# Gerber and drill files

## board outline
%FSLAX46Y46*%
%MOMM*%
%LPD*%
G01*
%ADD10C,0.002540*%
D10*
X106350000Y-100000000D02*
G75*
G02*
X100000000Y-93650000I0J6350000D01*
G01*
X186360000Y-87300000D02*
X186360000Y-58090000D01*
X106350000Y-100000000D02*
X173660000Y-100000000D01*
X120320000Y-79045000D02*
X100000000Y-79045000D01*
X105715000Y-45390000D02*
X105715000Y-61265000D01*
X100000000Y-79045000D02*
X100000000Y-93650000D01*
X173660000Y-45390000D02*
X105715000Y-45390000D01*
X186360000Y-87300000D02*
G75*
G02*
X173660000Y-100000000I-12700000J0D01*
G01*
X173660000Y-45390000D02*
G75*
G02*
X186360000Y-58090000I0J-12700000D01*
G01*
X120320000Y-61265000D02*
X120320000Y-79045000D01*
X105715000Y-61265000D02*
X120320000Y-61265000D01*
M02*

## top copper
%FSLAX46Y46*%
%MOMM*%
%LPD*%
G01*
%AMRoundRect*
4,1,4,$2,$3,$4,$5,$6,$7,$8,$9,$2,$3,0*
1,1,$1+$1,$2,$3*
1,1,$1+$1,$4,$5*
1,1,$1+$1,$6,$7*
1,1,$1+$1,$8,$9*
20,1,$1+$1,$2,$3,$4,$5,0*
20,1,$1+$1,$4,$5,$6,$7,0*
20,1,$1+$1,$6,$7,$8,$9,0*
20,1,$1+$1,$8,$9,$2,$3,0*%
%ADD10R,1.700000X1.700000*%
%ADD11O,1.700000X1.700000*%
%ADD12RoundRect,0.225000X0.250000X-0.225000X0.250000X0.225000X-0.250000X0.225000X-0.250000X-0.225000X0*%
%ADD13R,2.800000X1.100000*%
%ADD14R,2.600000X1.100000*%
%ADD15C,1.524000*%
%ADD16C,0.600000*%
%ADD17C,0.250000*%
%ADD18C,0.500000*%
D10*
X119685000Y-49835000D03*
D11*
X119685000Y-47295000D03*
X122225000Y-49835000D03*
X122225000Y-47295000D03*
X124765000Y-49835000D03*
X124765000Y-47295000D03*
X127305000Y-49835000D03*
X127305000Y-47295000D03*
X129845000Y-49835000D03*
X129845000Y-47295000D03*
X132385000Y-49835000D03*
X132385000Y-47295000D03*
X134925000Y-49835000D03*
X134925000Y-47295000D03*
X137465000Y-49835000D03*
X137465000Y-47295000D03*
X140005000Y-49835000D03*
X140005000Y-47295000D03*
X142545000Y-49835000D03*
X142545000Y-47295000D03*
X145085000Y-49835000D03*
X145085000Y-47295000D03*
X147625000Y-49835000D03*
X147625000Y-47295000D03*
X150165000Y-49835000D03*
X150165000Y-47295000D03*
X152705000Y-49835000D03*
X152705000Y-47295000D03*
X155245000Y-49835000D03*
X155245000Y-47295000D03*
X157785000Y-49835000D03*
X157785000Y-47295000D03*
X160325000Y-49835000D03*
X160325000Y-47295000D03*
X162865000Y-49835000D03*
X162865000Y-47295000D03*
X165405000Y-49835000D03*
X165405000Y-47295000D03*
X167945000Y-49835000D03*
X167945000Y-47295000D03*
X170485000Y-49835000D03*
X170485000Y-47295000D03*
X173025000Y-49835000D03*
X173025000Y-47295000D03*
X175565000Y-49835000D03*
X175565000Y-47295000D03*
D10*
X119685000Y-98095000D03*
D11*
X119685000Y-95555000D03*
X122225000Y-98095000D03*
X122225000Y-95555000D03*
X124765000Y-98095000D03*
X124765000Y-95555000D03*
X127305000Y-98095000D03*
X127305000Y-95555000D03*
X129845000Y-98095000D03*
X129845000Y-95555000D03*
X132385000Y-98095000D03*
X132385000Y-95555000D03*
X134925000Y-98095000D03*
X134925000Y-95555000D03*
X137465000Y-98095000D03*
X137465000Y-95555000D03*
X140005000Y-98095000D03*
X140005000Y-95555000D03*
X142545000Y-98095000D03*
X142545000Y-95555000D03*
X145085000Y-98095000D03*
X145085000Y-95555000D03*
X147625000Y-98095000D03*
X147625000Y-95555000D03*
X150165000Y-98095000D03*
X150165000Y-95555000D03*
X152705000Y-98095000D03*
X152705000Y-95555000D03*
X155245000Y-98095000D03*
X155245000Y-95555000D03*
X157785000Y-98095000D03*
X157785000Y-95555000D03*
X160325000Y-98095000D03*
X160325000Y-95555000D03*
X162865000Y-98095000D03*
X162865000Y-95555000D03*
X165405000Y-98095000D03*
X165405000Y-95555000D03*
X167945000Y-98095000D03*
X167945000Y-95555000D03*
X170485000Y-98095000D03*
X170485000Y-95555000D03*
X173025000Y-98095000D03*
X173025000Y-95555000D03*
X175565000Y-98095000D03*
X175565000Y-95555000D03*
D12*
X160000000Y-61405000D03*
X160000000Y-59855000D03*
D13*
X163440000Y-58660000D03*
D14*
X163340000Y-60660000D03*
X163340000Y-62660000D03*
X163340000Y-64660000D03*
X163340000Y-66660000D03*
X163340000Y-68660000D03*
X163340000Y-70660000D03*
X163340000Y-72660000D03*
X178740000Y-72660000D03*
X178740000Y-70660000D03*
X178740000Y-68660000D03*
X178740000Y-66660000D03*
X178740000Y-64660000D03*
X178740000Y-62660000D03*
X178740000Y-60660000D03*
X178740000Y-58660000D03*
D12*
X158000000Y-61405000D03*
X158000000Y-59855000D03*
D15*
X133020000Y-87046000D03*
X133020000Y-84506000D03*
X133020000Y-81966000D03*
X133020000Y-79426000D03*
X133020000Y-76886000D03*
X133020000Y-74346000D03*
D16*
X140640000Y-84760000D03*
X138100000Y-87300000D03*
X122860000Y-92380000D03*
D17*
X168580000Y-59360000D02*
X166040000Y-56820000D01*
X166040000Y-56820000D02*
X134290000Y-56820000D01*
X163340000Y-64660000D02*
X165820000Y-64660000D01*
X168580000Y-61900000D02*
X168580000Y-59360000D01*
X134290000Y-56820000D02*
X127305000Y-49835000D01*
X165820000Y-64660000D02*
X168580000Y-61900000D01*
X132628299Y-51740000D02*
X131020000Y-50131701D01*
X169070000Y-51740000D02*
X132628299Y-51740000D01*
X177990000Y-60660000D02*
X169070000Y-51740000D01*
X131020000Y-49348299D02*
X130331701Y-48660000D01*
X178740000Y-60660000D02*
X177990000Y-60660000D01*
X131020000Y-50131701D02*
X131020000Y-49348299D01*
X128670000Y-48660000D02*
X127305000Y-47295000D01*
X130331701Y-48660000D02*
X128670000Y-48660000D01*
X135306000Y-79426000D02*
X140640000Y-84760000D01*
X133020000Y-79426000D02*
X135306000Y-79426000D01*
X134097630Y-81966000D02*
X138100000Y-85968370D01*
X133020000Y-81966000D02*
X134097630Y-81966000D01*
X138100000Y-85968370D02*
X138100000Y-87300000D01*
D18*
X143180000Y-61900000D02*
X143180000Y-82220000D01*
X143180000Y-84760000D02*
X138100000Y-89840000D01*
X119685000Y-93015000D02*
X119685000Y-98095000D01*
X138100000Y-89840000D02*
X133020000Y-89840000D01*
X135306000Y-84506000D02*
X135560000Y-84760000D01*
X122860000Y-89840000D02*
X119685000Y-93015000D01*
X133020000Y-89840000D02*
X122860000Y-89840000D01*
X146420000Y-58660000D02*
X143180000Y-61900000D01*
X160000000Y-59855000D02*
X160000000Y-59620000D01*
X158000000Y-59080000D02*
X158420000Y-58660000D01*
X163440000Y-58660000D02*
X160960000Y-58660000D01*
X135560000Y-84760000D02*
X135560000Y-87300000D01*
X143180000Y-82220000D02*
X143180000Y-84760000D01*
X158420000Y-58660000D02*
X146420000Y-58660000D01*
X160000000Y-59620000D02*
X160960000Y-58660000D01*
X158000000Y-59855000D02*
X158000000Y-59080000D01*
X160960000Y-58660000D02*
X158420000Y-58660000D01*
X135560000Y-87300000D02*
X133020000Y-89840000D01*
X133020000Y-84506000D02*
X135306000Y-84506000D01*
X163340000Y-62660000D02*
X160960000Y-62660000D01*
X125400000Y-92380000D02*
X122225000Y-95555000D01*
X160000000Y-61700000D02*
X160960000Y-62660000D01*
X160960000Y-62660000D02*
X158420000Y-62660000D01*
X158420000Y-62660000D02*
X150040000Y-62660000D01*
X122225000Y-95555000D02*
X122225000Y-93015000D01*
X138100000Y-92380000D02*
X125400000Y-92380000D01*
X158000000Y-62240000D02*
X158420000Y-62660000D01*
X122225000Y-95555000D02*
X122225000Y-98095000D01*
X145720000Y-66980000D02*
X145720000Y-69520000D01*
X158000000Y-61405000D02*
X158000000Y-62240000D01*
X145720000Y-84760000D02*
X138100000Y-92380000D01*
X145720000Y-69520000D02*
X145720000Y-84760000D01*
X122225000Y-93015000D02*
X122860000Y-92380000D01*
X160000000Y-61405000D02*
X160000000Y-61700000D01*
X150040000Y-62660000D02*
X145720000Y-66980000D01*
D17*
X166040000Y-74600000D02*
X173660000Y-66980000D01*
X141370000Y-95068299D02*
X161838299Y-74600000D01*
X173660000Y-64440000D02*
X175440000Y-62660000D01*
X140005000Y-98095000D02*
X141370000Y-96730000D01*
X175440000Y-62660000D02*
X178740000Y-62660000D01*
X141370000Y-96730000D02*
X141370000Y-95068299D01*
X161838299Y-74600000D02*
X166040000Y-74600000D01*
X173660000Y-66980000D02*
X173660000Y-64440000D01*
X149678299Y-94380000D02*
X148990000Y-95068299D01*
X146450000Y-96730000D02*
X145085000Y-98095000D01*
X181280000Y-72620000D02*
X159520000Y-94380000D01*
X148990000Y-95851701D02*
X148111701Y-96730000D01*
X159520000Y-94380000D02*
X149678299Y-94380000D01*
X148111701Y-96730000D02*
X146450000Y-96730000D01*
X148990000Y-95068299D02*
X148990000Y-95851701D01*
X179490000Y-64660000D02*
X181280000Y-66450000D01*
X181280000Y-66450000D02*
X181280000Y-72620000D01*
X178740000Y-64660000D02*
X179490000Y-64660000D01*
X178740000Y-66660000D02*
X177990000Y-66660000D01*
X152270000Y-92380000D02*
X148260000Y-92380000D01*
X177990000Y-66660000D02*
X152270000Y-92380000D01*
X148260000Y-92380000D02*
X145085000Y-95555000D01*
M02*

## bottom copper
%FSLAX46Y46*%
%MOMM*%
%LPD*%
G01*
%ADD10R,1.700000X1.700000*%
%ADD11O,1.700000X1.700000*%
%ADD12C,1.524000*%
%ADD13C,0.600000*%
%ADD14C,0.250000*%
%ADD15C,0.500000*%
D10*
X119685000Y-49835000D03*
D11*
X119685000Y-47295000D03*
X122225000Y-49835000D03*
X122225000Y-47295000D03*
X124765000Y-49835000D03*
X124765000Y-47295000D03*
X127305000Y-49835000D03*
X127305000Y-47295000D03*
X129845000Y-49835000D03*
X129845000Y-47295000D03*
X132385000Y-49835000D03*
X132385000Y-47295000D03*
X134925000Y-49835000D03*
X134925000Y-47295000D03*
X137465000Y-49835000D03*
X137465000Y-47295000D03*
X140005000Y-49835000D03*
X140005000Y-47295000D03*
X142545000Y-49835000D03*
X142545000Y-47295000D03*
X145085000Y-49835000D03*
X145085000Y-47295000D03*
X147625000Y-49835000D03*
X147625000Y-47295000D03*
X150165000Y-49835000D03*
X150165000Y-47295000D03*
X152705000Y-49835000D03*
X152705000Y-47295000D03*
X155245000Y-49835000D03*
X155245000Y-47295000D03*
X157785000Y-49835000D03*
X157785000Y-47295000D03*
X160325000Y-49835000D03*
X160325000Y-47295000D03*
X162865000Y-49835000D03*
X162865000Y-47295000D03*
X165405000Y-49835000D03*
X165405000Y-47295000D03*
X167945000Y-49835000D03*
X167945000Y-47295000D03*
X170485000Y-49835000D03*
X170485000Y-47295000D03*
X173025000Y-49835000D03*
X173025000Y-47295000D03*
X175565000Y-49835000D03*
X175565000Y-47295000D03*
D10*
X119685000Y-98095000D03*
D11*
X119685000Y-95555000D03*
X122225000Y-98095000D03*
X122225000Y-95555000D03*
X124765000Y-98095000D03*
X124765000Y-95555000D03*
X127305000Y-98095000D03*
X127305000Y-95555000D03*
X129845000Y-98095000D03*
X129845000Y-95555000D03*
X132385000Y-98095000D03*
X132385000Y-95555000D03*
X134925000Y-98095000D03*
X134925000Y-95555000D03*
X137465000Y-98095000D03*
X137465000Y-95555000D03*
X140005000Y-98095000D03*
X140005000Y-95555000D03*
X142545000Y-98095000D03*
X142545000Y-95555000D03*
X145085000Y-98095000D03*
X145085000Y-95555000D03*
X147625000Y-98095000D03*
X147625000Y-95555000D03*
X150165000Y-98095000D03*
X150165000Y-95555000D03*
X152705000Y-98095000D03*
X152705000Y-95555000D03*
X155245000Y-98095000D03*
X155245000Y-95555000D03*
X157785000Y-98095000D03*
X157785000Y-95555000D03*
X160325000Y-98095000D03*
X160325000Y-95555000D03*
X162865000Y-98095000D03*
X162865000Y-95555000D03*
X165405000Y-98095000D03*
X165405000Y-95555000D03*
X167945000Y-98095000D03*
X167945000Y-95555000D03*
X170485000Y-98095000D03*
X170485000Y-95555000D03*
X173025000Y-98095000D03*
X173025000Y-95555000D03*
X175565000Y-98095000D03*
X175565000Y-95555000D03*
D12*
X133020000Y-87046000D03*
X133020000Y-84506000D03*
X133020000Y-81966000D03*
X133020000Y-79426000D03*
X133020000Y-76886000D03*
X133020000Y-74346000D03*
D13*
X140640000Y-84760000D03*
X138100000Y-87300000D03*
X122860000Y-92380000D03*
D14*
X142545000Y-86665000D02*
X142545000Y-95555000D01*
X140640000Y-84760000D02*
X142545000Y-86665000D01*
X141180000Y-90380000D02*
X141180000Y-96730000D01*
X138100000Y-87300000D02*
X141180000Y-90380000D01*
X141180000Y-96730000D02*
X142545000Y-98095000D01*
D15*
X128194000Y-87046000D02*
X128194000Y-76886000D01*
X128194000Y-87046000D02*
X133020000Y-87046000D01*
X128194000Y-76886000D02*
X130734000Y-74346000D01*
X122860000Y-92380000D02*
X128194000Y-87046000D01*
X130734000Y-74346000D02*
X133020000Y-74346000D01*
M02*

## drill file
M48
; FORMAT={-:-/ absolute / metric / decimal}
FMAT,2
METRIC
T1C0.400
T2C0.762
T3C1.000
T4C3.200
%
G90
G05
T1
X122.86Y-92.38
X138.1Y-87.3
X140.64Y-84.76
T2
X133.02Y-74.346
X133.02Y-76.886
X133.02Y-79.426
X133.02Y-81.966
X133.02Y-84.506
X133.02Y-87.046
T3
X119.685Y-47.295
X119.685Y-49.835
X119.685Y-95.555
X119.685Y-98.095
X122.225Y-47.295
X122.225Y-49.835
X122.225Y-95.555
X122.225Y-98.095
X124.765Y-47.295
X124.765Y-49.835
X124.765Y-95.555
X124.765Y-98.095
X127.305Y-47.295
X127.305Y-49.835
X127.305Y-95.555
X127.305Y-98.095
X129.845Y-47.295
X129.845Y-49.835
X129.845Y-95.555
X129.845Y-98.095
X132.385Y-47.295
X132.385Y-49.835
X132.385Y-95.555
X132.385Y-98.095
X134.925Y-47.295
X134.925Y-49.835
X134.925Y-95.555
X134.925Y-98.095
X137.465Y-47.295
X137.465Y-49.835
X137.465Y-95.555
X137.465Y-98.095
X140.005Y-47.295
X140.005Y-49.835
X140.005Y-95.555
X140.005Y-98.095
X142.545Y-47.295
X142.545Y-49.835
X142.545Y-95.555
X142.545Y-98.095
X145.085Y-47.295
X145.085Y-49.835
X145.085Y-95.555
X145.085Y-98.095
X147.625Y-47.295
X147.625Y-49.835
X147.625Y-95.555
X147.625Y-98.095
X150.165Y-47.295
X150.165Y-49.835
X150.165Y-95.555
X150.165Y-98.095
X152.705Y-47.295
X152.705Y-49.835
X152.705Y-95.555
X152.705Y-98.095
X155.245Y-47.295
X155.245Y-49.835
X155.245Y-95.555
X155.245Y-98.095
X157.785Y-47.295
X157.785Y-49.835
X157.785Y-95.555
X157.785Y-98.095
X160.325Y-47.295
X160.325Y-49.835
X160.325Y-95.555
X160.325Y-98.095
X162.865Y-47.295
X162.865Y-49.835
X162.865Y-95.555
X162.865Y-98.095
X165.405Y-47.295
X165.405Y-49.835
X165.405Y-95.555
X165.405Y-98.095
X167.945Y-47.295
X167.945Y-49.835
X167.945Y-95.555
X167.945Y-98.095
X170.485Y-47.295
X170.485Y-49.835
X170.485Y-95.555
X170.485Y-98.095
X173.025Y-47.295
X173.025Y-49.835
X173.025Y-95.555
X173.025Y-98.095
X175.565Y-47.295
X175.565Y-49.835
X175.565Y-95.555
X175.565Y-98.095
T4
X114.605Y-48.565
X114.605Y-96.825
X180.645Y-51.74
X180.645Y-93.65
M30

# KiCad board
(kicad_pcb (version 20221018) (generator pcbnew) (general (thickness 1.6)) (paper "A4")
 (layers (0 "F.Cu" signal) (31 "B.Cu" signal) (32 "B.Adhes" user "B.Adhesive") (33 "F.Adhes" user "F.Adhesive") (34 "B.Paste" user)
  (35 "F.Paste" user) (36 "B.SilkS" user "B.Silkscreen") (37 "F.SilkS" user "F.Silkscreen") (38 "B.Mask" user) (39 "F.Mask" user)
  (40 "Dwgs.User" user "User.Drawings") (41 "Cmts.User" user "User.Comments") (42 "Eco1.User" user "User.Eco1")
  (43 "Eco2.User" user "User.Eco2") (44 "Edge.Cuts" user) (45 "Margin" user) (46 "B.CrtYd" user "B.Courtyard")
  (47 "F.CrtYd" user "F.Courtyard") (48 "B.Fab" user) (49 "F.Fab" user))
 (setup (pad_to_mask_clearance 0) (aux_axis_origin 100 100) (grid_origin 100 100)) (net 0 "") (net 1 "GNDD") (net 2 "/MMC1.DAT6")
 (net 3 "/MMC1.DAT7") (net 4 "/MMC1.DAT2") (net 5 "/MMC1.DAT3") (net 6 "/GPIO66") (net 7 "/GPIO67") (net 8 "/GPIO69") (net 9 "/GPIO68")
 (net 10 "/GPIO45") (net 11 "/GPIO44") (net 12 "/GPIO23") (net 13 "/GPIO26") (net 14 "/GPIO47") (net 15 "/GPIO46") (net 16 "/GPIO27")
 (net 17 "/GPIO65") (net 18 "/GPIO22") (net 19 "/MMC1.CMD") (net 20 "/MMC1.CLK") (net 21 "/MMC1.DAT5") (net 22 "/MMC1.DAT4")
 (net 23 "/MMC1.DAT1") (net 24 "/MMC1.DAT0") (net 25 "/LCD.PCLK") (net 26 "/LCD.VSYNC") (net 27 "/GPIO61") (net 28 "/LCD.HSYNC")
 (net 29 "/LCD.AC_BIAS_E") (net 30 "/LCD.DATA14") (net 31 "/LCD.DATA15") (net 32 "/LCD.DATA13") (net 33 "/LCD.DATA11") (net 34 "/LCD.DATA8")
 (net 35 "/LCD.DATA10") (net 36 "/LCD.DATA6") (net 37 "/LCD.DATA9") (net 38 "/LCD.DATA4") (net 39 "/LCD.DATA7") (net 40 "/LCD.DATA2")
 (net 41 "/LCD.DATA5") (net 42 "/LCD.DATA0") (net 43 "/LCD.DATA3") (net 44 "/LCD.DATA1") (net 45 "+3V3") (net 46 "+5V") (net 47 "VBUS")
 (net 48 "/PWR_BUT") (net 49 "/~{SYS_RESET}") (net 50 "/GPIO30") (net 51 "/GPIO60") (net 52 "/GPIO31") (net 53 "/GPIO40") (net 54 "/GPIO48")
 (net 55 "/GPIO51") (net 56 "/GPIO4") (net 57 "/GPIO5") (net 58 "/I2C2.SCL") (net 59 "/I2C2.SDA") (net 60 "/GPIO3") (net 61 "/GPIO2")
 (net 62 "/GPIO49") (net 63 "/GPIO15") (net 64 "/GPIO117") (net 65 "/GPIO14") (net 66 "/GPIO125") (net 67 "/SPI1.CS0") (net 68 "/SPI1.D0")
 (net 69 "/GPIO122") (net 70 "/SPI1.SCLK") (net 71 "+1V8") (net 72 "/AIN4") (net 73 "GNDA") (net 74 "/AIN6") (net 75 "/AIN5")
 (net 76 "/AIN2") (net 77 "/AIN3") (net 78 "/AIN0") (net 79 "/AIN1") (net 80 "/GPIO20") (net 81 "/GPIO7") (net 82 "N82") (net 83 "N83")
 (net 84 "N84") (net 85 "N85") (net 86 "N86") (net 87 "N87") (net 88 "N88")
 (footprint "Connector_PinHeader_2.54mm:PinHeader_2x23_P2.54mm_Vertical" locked (layer "F.Cu") (at 119.685 49.835 90)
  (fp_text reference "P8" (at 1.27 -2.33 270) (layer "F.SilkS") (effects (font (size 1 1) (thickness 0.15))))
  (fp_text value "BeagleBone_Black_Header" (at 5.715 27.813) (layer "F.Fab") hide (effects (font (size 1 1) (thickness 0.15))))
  (pad "1" thru_hole rect locked (at 0 0 90) (size 1.7 1.7) (drill 1) (layers "*.Cu" "*.Mask") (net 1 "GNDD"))
  (pad "2" thru_hole oval locked (at 2.54 0 90) (size 1.7 1.7) (drill 1) (layers "*.Cu" "*.Mask") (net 1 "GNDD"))
  (pad "3" thru_hole oval locked (at 0 2.54 90) (size 1.7 1.7) (drill 1) (layers "*.Cu" "*.Mask") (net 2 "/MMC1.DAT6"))
  (pad "4" thru_hole oval locked (at 2.54 2.54 90) (size 1.7 1.7) (drill 1) (layers "*.Cu" "*.Mask") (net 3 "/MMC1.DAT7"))
  (pad "5" thru_hole oval locked (at 0 5.08 90) (size 1.7 1.7) (drill 1) (layers "*.Cu" "*.Mask") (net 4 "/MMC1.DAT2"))
  (pad "6" thru_hole oval locked (at 2.54 5.08 90) (size 1.7 1.7) (drill 1) (layers "*.Cu" "*.Mask") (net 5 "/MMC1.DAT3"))
  (pad "7" thru_hole oval locked (at 0 7.62 90) (size 1.7 1.7) (drill 1) (layers "*.Cu" "*.Mask") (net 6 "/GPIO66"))
  (pad "8" thru_hole oval locked (at 2.54 7.62 90) (size 1.7 1.7) (drill 1) (layers "*.Cu" "*.Mask") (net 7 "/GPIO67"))
  (pad "9" thru_hole oval locked (at 0 10.16 90) (size 1.7 1.7) (drill 1) (layers "*.Cu" "*.Mask") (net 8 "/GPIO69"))
  (pad "10" thru_hole oval locked (at 2.54 10.16 90) (size 1.7 1.7) (drill 1) (layers "*.Cu" "*.Mask") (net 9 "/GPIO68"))
  (pad "11" thru_hole oval locked (at 0 12.7 90) (size 1.7 1.7) (drill 1) (layers "*.Cu" "*.Mask") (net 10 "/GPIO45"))
  (pad "12" thru_hole oval locked (at 2.54 12.7 90) (size 1.7 1.7) (drill 1) (layers "*.Cu" "*.Mask") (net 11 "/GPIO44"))
  (pad "13" thru_hole oval locked (at 0 15.24 90) (size 1.7 1.7) (drill 1) (layers "*.Cu" "*.Mask") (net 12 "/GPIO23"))
  (pad "14" thru_hole oval locked (at 2.54 15.24 90) (size 1.7 1.7) (drill 1) (layers "*.Cu" "*.Mask") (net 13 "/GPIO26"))
  (pad "15" thru_hole oval locked (at 0 17.78 90) (size 1.7 1.7) (drill 1) (layers "*.Cu" "*.Mask") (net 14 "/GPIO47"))
  (pad "16" thru_hole oval locked (at 2.54 17.78 90) (size 1.7 1.7) (drill 1) (layers "*.Cu" "*.Mask") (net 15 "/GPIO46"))
  (pad "17" thru_hole oval locked (at 0 20.32 90) (size 1.7 1.7) (drill 1) (layers "*.Cu" "*.Mask") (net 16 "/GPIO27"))
  (pad "18" thru_hole oval locked (at 2.54 20.32 90) (size 1.7 1.7) (drill 1) (layers "*.Cu" "*.Mask") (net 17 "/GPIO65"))
  (pad "19" thru_hole oval locked (at 0 22.86 90) (size 1.7 1.7) (drill 1) (layers "*.Cu" "*.Mask") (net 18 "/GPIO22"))
  (pad "20" thru_hole oval locked (at 2.54 22.86 90) (size 1.7 1.7) (drill 1) (layers "*.Cu" "*.Mask") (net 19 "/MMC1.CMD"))
  (pad "21" thru_hole oval locked (at 0 25.4 90) (size 1.7 1.7) (drill 1) (layers "*.Cu" "*.Mask") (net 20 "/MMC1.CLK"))
  (pad "22" thru_hole oval locked (at 2.54 25.4 90) (size 1.7 1.7) (drill 1) (layers "*.Cu" "*.Mask") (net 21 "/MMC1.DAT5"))
  (pad "23" thru_hole oval locked (at 0 27.94 90) (size 1.7 1.7) (drill 1) (layers "*.Cu" "*.Mask") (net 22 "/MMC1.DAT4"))
  (pad "24" thru_hole oval locked (at 2.54 27.94 90) (size 1.7 1.7) (drill 1) (layers "*.Cu" "*.Mask") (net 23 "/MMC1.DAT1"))
  (pad "25" thru_hole oval locked (at 0 30.48 90) (size 1.7 1.7) (drill 1) (layers "*.Cu" "*.Mask") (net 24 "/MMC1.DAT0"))
  (pad "26" thru_hole oval locked (at 2.54 30.48 90) (size 1.7 1.7) (drill 1) (layers "*.Cu" "*.Mask") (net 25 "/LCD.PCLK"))
  (pad "27" thru_hole oval locked (at 0 33.02 90) (size 1.7 1.7) (drill 1) (layers "*.Cu" "*.Mask") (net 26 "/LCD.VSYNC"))
  (pad "28" thru_hole oval locked (at 2.54 33.02 90) (size 1.7 1.7) (drill 1) (layers "*.Cu" "*.Mask") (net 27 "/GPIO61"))
  (pad "29" thru_hole oval locked (at 0 35.56 90) (size 1.7 1.7) (drill 1) (layers "*.Cu" "*.Mask") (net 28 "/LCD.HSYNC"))
  (pad "30" thru_hole oval locked (at 2.54 35.56 90) (size 1.7 1.7) (drill 1) (layers "*.Cu" "*.Mask") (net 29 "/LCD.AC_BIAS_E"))
  (pad "31" thru_hole oval locked (at 0 38.1 90) (size 1.7 1.7) (drill 1) (layers "*.Cu" "*.Mask") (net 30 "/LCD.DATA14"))
  (pad "32" thru_hole oval locked (at 2.54 38.1 90) (size 1.7 1.7) (drill 1) (layers "*.Cu" "*.Mask") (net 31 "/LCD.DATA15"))
  (pad "33" thru_hole oval locked (at 0 40.64 90) (size 1.7 1.7) (drill 1) (layers "*.Cu" "*.Mask") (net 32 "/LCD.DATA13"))
  (pad "34" thru_hole oval locked (at 2.54 40.64 90) (size 1.7 1.7) (drill 1) (layers "*.Cu" "*.Mask") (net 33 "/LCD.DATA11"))
  (pad "35" thru_hole oval locked (at 0 43.18 90) (size 1.7 1.7) (drill 1) (layers "*.Cu" "*.Mask") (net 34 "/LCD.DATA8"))
  (pad "36" thru_hole oval locked (at 2.54 43.18 90) (size 1.7 1.7) (drill 1) (layers "*.Cu" "*.Mask") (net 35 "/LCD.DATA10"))
  (pad "37" thru_hole oval locked (at 0 45.72 90) (size 1.7 1.7) (drill 1) (layers "*.Cu" "*.Mask") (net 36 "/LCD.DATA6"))
  (pad "38" thru_hole oval locked (at 2.54 45.72 90) (size 1.7 1.7) (drill 1) (layers "*.Cu" "*.Mask") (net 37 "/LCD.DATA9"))
  (pad "39" thru_hole oval locked (at 0 48.26 90) (size 1.7 1.7) (drill 1) (layers "*.Cu" "*.Mask") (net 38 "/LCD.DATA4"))
  (pad "40" thru_hole oval locked (at 2.54 48.26 90) (size 1.7 1.7) (drill 1) (layers "*.Cu" "*.Mask") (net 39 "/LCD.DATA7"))
  (pad "41" thru_hole oval locked (at 0 50.8 90) (size 1.7 1.7) (drill 1) (layers "*.Cu" "*.Mask") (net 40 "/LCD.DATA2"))
  (pad "42" thru_hole oval locked (at 2.54 50.8 90) (size 1.7 1.7) (drill 1) (layers "*.Cu" "*.Mask") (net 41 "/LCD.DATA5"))
  (pad "43" thru_hole oval locked (at 0 53.34 90) (size 1.7 1.7) (drill 1) (layers "*.Cu" "*.Mask") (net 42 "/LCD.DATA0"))
  (pad "44" thru_hole oval locked (at 2.54 53.34 90) (size 1.7 1.7) (drill 1) (layers "*.Cu" "*.Mask") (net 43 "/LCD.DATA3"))
  (pad "45" thru_hole oval locked (at 0 55.88 90) (size 1.7 1.7) (drill 1) (layers "*.Cu" "*.Mask") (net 1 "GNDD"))
  (pad "46" thru_hole oval locked (at 2.54 55.88 90) (size 1.7 1.7) (drill 1) (layers "*.Cu" "*.Mask") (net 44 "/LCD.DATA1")))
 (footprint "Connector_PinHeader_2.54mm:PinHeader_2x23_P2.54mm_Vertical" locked (layer "F.Cu") (at 119.685 98.095 90)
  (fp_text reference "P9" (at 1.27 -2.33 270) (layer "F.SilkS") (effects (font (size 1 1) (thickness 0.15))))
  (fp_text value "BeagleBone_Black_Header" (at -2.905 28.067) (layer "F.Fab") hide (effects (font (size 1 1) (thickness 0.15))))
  (pad "1" thru_hole rect locked (at 0 0 90) (size 1.7 1.7) (drill 1) (layers "*.Cu" "*.Mask") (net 1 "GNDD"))
  (pad "2" thru_hole oval locked (at 2.54 0 90) (size 1.7 1.7) (drill 1) (layers "*.Cu" "*.Mask") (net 1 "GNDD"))
  (pad "3" thru_hole oval locked (at 0 2.54 90) (size 1.7 1.7) (drill 1) (layers "*.Cu" "*.Mask") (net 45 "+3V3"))
  (pad "4" thru_hole oval locked (at 2.54 2.54 90) (size 1.7 1.7) (drill 1) (layers "*.Cu" "*.Mask") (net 45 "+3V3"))
  (pad "5" thru_hole oval locked (at 0 5.08 90) (size 1.7 1.7) (drill 1) (layers "*.Cu" "*.Mask") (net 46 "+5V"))
  (pad "6" thru_hole oval locked (at 2.54 5.08 90) (size 1.7 1.7) (drill 1) (layers "*.Cu" "*.Mask") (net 46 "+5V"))
  (pad "7" thru_hole oval locked (at 0 7.62 90) (size 1.7 1.7) (drill 1) (layers "*.Cu" "*.Mask") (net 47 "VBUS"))
  (pad "8" thru_hole oval locked (at 2.54 7.62 90) (size 1.7 1.7) (drill 1) (layers "*.Cu" "*.Mask") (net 47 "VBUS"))
  (pad "9" thru_hole oval locked (at 0 10.16 90) (size 1.7 1.7) (drill 1) (layers "*.Cu" "*.Mask") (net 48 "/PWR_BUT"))
  (pad "10" thru_hole oval locked (at 2.54 10.16 90) (size 1.7 1.7) (drill 1) (layers "*.Cu" "*.Mask") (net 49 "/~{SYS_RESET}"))
  (pad "11" thru_hole oval locked (at 0 12.7 90) (size 1.7 1.7) (drill 1) (layers "*.Cu" "*.Mask") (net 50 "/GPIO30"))
  (pad "12" thru_hole oval locked (at 2.54 12.7 90) (size 1.7 1.7) (drill 1) (layers "*.Cu" "*.Mask") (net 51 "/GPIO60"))
  (pad "13" thru_hole oval locked (at 0 15.24 90) (size 1.7 1.7) (drill 1) (layers "*.Cu" "*.Mask") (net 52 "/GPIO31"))
  (pad "14" thru_hole oval locked (at 2.54 15.24 90) (size 1.7 1.7) (drill 1) (layers "*.Cu" "*.Mask") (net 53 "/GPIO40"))
  (pad "15" thru_hole oval locked (at 0 17.78 90) (size 1.7 1.7) (drill 1) (layers "*.Cu" "*.Mask") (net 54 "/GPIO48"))
  (pad "16" thru_hole oval locked (at 2.54 17.78 90) (size 1.7 1.7) (drill 1) (layers "*.Cu" "*.Mask") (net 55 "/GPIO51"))
  (pad "17" thru_hole oval locked (at 0 20.32 90) (size 1.7 1.7) (drill 1) (layers "*.Cu" "*.Mask") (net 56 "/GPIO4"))
  (pad "18" thru_hole oval locked (at 2.54 20.32 90) (size 1.7 1.7) (drill 1) (layers "*.Cu" "*.Mask") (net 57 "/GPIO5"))
  (pad "19" thru_hole oval locked (at 0 22.86 90) (size 1.7 1.7) (drill 1) (layers "*.Cu" "*.Mask") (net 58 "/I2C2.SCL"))
  (pad "20" thru_hole oval locked (at 2.54 22.86 90) (size 1.7 1.7) (drill 1) (layers "*.Cu" "*.Mask") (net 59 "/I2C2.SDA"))
  (pad "21" thru_hole oval locked (at 0 25.4 90) (size 1.7 1.7) (drill 1) (layers "*.Cu" "*.Mask") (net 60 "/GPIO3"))
  (pad "22" thru_hole oval locked (at 2.54 25.4 90) (size 1.7 1.7) (drill 1) (layers "*.Cu" "*.Mask") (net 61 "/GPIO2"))
  (pad "23" thru_hole oval locked (at 0 27.94 90) (size 1.7 1.7) (drill 1) (layers "*.Cu" "*.Mask") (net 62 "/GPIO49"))
  (pad "24" thru_hole oval locked (at 2.54 27.94 90) (size 1.7 1.7) (drill 1) (layers "*.Cu" "*.Mask") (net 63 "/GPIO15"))
  (pad "25" thru_hole oval locked (at 0 30.48 90) (size 1.7 1.7) (drill 1) (layers "*.Cu" "*.Mask") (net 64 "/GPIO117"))
  (pad "26" thru_hole oval locked (at 2.54 30.48 90) (size 1.7 1.7) (drill 1) (layers "*.Cu" "*.Mask") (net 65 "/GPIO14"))
  (pad "27" thru_hole oval locked (at 0 33.02 90) (size 1.7 1.7) (drill 1) (layers "*.Cu" "*.Mask") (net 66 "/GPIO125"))
  (pad "28" thru_hole oval locked (at 2.54 33.02 90) (size 1.7 1.7) (drill 1) (layers "*.Cu" "*.Mask") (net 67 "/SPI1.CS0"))
  (pad "29" thru_hole oval locked (at 0 35.56 90) (size 1.7 1.7) (drill 1) (layers "*.Cu" "*.Mask") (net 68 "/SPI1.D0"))
  (pad "30" thru_hole oval locked (at 2.54 35.56 90) (size 1.7 1.7) (drill 1) (layers "*.Cu" "*.Mask") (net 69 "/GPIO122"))
  (pad "31" thru_hole oval locked (at 0 38.1 90) (size 1.7 1.7) (drill 1) (layers "*.Cu" "*.Mask") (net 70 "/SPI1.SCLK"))
  (pad "32" thru_hole oval locked (at 2.54 38.1 90) (size 1.7 1.7) (drill 1) (layers "*.Cu" "*.Mask") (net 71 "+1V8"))
  (pad "33" thru_hole oval locked (at 0 40.64 90) (size 1.7 1.7) (drill 1) (layers "*.Cu" "*.Mask") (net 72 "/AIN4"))
  (pad "34" thru_hole oval locked (at 2.54 40.64 90) (size 1.7 1.7) (drill 1) (layers "*.Cu" "*.Mask") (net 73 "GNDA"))
  (pad "35" thru_hole oval locked (at 0 43.18 90) (size 1.7 1.7) (drill 1) (layers "*.Cu" "*.Mask") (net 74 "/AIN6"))
  (pad "36" thru_hole oval locked (at 2.54 43.18 90) (size 1.7 1.7) (drill 1) (layers "*.Cu" "*.Mask") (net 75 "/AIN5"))
  (pad "37" thru_hole oval locked (at 0 45.72 90) (size 1.7 1.7) (drill 1) (layers "*.Cu" "*.Mask") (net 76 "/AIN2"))
  (pad "38" thru_hole oval locked (at 2.54 45.72 90) (size 1.7 1.7) (drill 1) (layers "*.Cu" "*.Mask") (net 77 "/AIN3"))
  (pad "39" thru_hole oval locked (at 0 48.26 90) (size 1.7 1.7) (drill 1) (layers "*.Cu" "*.Mask") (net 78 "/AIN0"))
  (pad "40" thru_hole oval locked (at 2.54 48.26 90) (size 1.7 1.7) (drill 1) (layers "*.Cu" "*.Mask") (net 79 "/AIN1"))
  (pad "41" thru_hole oval locked (at 0 50.8 90) (size 1.7 1.7) (drill 1) (layers "*.Cu" "*.Mask") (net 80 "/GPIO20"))
  (pad "42" thru_hole oval locked (at 2.54 50.8 90) (size 1.7 1.7) (drill 1) (layers "*.Cu" "*.Mask") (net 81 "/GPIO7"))
  (pad "43" thru_hole oval locked (at 0 53.34 90) (size 1.7 1.7) (drill 1) (layers "*.Cu" "*.Mask") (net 1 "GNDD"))
  (pad "44" thru_hole oval locked (at 2.54 53.34 90) (size 1.7 1.7) (drill 1) (layers "*.Cu" "*.Mask") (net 1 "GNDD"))
  (pad "45" thru_hole oval locked (at 0 55.88 90) (size 1.7 1.7) (drill 1) (layers "*.Cu" "*.Mask") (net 1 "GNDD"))
  (pad "46" thru_hole oval locked (at 2.54 55.88 90) (size 1.7 1.7) (drill 1) (layers "*.Cu" "*.Mask") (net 1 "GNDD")))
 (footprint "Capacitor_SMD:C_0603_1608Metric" (layer "F.Cu") (at 160 60.63 90)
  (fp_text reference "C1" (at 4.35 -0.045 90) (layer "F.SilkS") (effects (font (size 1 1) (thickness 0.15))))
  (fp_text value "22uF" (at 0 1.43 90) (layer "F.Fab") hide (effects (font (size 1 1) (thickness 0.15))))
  (pad "1" smd roundrect (at -0.775 0 90) (size 0.9 0.95) (layers "F.Cu" "F.Paste" "F.Mask") (roundrect_rratio 0.25) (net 45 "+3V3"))
  (pad "2" smd roundrect (at 0.775 0 90) (size 0.9 0.95) (layers "F.Cu" "F.Paste" "F.Mask") (roundrect_rratio 0.25) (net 1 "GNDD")))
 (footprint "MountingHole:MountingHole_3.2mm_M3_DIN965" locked (layer "F.Cu") (at 180.645 51.74)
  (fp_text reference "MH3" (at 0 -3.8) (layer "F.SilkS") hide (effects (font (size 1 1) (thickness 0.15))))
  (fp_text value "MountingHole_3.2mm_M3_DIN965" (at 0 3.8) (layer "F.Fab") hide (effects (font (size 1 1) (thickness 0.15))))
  (pad "" np_thru_hole circle locked (at 0 0) (size 3.2 3.2) (drill 3.2) (layers "*.Cu" "*.Mask")))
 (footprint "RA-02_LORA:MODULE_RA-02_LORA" (layer "F.Cu") (at 171.04 65.66)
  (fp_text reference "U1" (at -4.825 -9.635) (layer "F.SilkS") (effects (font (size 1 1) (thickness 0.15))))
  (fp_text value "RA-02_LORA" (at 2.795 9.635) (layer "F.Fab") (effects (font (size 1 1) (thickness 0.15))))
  (pad "1" smd rect (at -7.6 -7) (size 2.8 1.1) (layers "F.Cu" "F.Paste" "F.Mask") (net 1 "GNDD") (solder_mask_margin 0.102))
  (pad "2" smd rect (at -7.7 -5) (size 2.6 1.1) (layers "F.Cu" "F.Paste" "F.Mask") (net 1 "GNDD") (solder_mask_margin 0.102))
  (pad "3" smd rect (at -7.7 -3) (size 2.6 1.1) (layers "F.Cu" "F.Paste" "F.Mask") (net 45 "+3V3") (solder_mask_margin 0.102))
  (pad "4" smd rect (at -7.7 -1) (size 2.6 1.1) (layers "F.Cu" "F.Paste" "F.Mask") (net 6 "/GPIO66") (solder_mask_margin 0.102))
  (pad "5" smd rect (at -7.7 1) (size 2.6 1.1) (layers "F.Cu" "F.Paste" "F.Mask") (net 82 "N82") (solder_mask_margin 0.102))
  (pad "6" smd rect (at -7.7 3) (size 2.6 1.1) (layers "F.Cu" "F.Paste" "F.Mask") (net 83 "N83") (solder_mask_margin 0.102))
  (pad "7" smd rect (at -7.7 5) (size 2.6 1.1) (layers "F.Cu" "F.Paste" "F.Mask") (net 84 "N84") (solder_mask_margin 0.102))
  (pad "8" smd rect (at -7.7 7) (size 2.6 1.1) (layers "F.Cu" "F.Paste" "F.Mask") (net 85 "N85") (solder_mask_margin 0.102))
  (pad "9" smd rect (at 7.7 7 180) (size 2.6 1.1) (layers "F.Cu" "F.Paste" "F.Mask") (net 1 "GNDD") (solder_mask_margin 0.102))
  (pad "10" smd rect (at 7.7 5 180) (size 2.6 1.1) (layers "F.Cu" "F.Paste" "F.Mask") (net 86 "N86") (solder_mask_margin 0.102))
  (pad "11" smd rect (at 7.7 3 180) (size 2.6 1.1) (layers "F.Cu" "F.Paste" "F.Mask") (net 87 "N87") (solder_mask_margin 0.102))
  (pad "12" smd rect (at 7.7 1 180) (size 2.6 1.1) (layers "F.Cu" "F.Paste" "F.Mask") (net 61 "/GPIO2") (solder_mask_margin 0.102))
  (pad "13" smd rect (at 7.7 -1 180) (size 2.6 1.1) (layers "F.Cu" "F.Paste" "F.Mask") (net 60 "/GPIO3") (solder_mask_margin 0.102))
  (pad "14" smd rect (at 7.7 -3 180) (size 2.6 1.1) (layers "F.Cu" "F.Paste" "F.Mask") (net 56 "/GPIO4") (solder_mask_margin 0.102))
  (pad "15" smd rect (at 7.7 -5 180) (size 2.6 1.1) (layers "F.Cu" "F.Paste" "F.Mask") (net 7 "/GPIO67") (solder_mask_margin 0.102))
  (pad "16" smd rect (at 7.7 -7 180) (size 2.6 1.1) (layers "F.Cu" "F.Paste" "F.Mask") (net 1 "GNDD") (solder_mask_margin 0.102)))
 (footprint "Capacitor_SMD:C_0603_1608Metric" (layer "F.Cu") (at 158 60.63 90)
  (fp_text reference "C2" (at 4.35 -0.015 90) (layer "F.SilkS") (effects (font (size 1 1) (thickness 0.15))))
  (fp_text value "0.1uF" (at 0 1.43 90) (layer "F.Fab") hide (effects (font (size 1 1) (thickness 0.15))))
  (pad "1" smd roundrect (at -0.775 0 90) (size 0.9 0.95) (layers "F.Cu" "F.Paste" "F.Mask") (roundrect_rratio 0.25) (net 45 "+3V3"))
  (pad "2" smd roundrect (at 0.775 0 90) (size 0.9 0.95) (layers "F.Cu" "F.Paste" "F.Mask") (roundrect_rratio 0.25) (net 1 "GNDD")))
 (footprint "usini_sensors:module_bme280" (layer "F.Cu") (at 127.94 74.6 180)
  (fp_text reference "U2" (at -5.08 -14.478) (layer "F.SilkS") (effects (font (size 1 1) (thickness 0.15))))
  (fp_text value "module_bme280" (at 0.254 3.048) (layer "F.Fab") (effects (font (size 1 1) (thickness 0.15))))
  (pad "1" thru_hole circle (at -5.08 -12.446 180) (size 1.524 1.524) (drill 0.762) (layers "*.Cu" "*.Mask") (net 45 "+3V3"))
  (pad "2" thru_hole circle (at -5.08 -9.906 180) (size 1.524 1.524) (drill 0.762) (layers "*.Cu" "*.Mask") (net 1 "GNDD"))
  (pad "3" thru_hole circle (at -5.08 -7.366 180) (size 1.524 1.524) (drill 0.762) (layers "*.Cu" "*.Mask") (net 58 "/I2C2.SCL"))
  (pad "4" thru_hole circle (at -5.08 -4.826 180) (size 1.524 1.524) (drill 0.762) (layers "*.Cu" "*.Mask") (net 59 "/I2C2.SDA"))
  (pad "5" thru_hole circle (at -5.08 -2.286 180) (size 1.524 1.524) (drill 0.762) (layers "*.Cu" "*.Mask") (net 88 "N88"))
  (pad "6" thru_hole circle (at -5.08 0.254 180) (size 1.524 1.524) (drill 0.762) (layers "*.Cu" "*.Mask") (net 45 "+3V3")))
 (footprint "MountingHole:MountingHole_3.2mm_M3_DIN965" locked (layer "F.Cu") (at 180.645 93.65)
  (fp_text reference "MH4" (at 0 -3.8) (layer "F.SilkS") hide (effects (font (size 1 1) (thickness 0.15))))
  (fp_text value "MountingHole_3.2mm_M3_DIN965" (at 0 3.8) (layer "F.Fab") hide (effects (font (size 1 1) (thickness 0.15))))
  (pad "" np_thru_hole circle locked (at 0 0) (size 3.2 3.2) (drill 3.2) (layers "*.Cu" "*.Mask")))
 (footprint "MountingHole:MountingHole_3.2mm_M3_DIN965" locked (layer "F.Cu") (at 114.605 48.565)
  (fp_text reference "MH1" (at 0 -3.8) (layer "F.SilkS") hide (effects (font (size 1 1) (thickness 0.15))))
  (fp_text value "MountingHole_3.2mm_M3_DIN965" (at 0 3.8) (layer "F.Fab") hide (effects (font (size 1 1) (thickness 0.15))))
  (pad "" np_thru_hole circle locked (at 0 0) (size 3.2 3.2) (drill 3.2) (layers "*.Cu" "*.Mask")))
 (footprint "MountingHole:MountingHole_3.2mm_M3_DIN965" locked (layer "F.Cu") (at 114.605 96.825)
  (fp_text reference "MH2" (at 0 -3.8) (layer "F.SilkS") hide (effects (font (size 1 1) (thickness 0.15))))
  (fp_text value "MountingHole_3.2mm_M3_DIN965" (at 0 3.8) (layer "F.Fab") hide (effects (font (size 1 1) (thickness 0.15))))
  (pad "" np_thru_hole circle locked (at 0 0) (size 3.2 3.2) (drill 3.2) (layers "*.Cu" "*.Mask")))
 (gr_arc locked (start 106.35 100) (mid 101.859872 98.140128) (end 100 93.65) (stroke (width 0.00254) (type solid)) (layer "Edge.Cuts"))
 (gr_line locked (start 186.36 87.3) (end 186.36 58.09) (stroke (width 0.00254) (type solid)) (layer "Edge.Cuts"))
 (gr_line locked (start 106.35 100) (end 173.66 100) (stroke (width 0.00254) (type solid)) (layer "Edge.Cuts"))
 (gr_line locked (start 120.32 79.045) (end 100 79.045) (stroke (width 0.00254) (type solid)) (layer "Edge.Cuts"))
 (gr_line locked (start 105.715 45.39) (end 105.715 61.265) (stroke (width 0.00254) (type solid)) (layer "Edge.Cuts"))
 (gr_line locked (start 100 79.045) (end 100 93.65) (stroke (width 0.00254) (type solid)) (layer "Edge.Cuts"))
 (gr_line locked (start 173.66 45.39) (end 105.715 45.39) (stroke (width 0.00254) (type solid)) (layer "Edge.Cuts"))
 (gr_arc locked (start 186.36 87.3) (mid 182.640256 96.280256) (end 173.66 100) (stroke (width 0.00254) (type solid)) (layer "Edge.Cuts"))
 (gr_arc locked (start 173.66 45.39) (mid 182.640256 49.109744) (end 186.36 58.09) (stroke (width 0.00254) (type solid)) (layer "Edge.Cuts"))
 (gr_line locked (start 120.32 61.265) (end 120.32 79.045) (stroke (width 0.00254) (type solid)) (layer "Edge.Cuts"))
 (gr_line locked (start 105.715 61.265) (end 120.32 61.265) (stroke (width 0.00254) (type solid)) (layer "Edge.Cuts"))
 (segment (start 168.58 59.36) (end 166.04 56.82) (width 0.25) (layer "F.Cu") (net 6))
 (segment (start 166.04 56.82) (end 134.29 56.82) (width 0.25) (layer "F.Cu") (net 6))
 (segment (start 163.34 64.66) (end 165.82 64.66) (width 0.25) (layer "F.Cu") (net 6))
 (segment (start 168.58 61.9) (end 168.58 59.36) (width 0.25) (layer "F.Cu") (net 6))
 (segment (start 134.29 56.82) (end 127.305 49.835) (width 0.25) (layer "F.Cu") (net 6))
 (segment (start 165.82 64.66) (end 168.58 61.9) (width 0.25) (layer "F.Cu") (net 6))
 (segment (start 132.628299 51.74) (end 131.02 50.131701) (width 0.25) (layer "F.Cu") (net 7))
 (segment (start 169.07 51.74) (end 132.628299 51.74) (width 0.25) (layer "F.Cu") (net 7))
 (segment (start 177.99 60.66) (end 169.07 51.74) (width 0.25) (layer "F.Cu") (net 7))
 (segment (start 131.02 49.348299) (end 130.331701 48.66) (width 0.25) (layer "F.Cu") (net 7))
 (segment (start 178.74 60.66) (end 177.99 60.66) (width 0.25) (layer "F.Cu") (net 7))
 (segment (start 131.02 50.131701) (end 131.02 49.348299) (width 0.25) (layer "F.Cu") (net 7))
 (segment (start 128.67 48.66) (end 127.305 47.295) (width 0.25) (layer "F.Cu") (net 7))
 (segment (start 130.331701 48.66) (end 128.67 48.66) (width 0.25) (layer "F.Cu") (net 7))
 (segment (start 135.306 79.426) (end 140.64 84.76) (width 0.25) (layer "F.Cu") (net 59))
 (segment (start 133.02 79.426) (end 135.306 79.426) (width 0.25) (layer "F.Cu") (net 59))
 (via (at 140.64 84.76) (size 0.6) (drill 0.4) (layers "F.Cu" "B.Cu") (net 59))
 (segment (start 142.545 86.665) (end 142.545 95.555) (width 0.25) (layer "B.Cu") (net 59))
 (segment (start 140.64 84.76) (end 142.545 86.665) (width 0.25) (layer "B.Cu") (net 59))
 (segment (start 134.09763 81.966) (end 138.1 85.96837) (width 0.25) (layer "F.Cu") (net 58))
 (segment (start 133.02 81.966) (end 134.09763 81.966) (width 0.25) (layer "F.Cu") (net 58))
 (segment (start 138.1 85.96837) (end 138.1 87.3) (width 0.25) (layer "F.Cu") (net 58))
 (via (at 138.1 87.3) (size 0.6) (drill 0.4) (layers "F.Cu" "B.Cu") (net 58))
 (segment (start 141.18 90.38) (end 141.18 96.73) (width 0.25) (layer "B.Cu") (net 58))
 (segment (start 138.1 87.3) (end 141.18 90.38) (width 0.25) (layer "B.Cu") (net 58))
 (segment (start 141.18 96.73) (end 142.545 98.095) (width 0.25) (layer "B.Cu") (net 58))
 (segment (start 143.18 61.9) (end 143.18 82.22) (width 0.5) (layer "F.Cu") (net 1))
 (segment (start 143.18 84.76) (end 138.1 89.84) (width 0.5) (layer "F.Cu") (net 1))
 (segment (start 119.685 93.015) (end 119.685 98.095) (width 0.5) (layer "F.Cu") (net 1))
 (segment (start 138.1 89.84) (end 133.02 89.84) (width 0.5) (layer "F.Cu") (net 1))
 (segment (start 135.306 84.506) (end 135.56 84.76) (width 0.5) (layer "F.Cu") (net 1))
 (segment (start 122.86 89.84) (end 119.685 93.015) (width 0.5) (layer "F.Cu") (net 1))
 (segment (start 133.02 89.84) (end 122.86 89.84) (width 0.5) (layer "F.Cu") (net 1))
 (segment (start 146.42 58.66) (end 143.18 61.9) (width 0.5) (layer "F.Cu") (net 1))
 (segment (start 160 59.855) (end 160 59.62) (width 0.5) (layer "F.Cu") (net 1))
 (segment (start 158 59.08) (end 158.42 58.66) (width 0.5) (layer "F.Cu") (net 1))
 (segment (start 163.44 58.66) (end 160.96 58.66) (width 0.5) (layer "F.Cu") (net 1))
 (segment (start 135.56 84.76) (end 135.56 87.3) (width 0.5) (layer "F.Cu") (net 1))
 (segment (start 143.18 82.22) (end 143.18 84.76) (width 0.5) (layer "F.Cu") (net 1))
 (segment (start 158.42 58.66) (end 146.42 58.66) (width 0.5) (layer "F.Cu") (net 1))
 (segment (start 160 59.62) (end 160.96 58.66) (width 0.5) (layer "F.Cu") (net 1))
 (segment (start 158 59.855) (end 158 59.08) (width 0.5) (layer "F.Cu") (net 1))
 (segment (start 160.96 58.66) (end 158.42 58.66) (width 0.5) (layer "F.Cu") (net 1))
 (segment (start 135.56 87.3) (end 133.02 89.84) (width 0.5) (layer "F.Cu") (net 1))
 (segment (start 133.02 84.506) (end 135.306 84.506) (width 0.5) (layer "F.Cu") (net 1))
 (segment (start 163.34 62.66) (end 160.96 62.66) (width 0.5) (layer "F.Cu") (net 45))
 (segment (start 125.4 92.38) (end 122.225 95.555) (width 0.5) (layer "F.Cu") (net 45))
 (segment (start 160 61.7) (end 160.96 62.66) (width 0.5) (layer "F.Cu") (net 45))
 (segment (start 160.96 62.66) (end 158.42 62.66) (width 0.5) (layer "F.Cu") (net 45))
 (segment (start 158.42 62.66) (end 150.04 62.66) (width 0.5) (layer "F.Cu") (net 45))
 (segment (start 122.225 95.555) (end 122.225 93.015) (width 0.5) (layer "F.Cu") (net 45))
 (segment (start 138.1 92.38) (end 125.4 92.38) (width 0.5) (layer "F.Cu") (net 45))
 (segment (start 158 62.24) (end 158.42 62.66) (width 0.5) (layer "F.Cu") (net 45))
 (segment (start 122.225 95.555) (end 122.225 98.095) (width 0.5) (layer "F.Cu") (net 45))
 (segment (start 145.72 66.98) (end 145.72 69.52) (width 0.5) (layer "F.Cu") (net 45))
 (segment (start 158 61.405) (end 158 62.24) (width 0.5) (layer "F.Cu") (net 45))
 (segment (start 145.72 84.76) (end 138.1 92.38) (width 0.5) (layer "F.Cu") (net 45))
 (segment (start 145.72 69.52) (end 145.72 84.76) (width 0.5) (layer "F.Cu") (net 45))
 (segment (start 122.225 93.015) (end 122.86 92.38) (width 0.5) (layer "F.Cu") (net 45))
 (segment (start 160 61.405) (end 160 61.7) (width 0.5) (layer "F.Cu") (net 45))
 (segment (start 150.04 62.66) (end 145.72 66.98) (width 0.5) (layer "F.Cu") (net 45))
 (via (at 122.86 92.38) (size 0.6) (drill 0.4) (layers "F.Cu" "B.Cu") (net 45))
 (segment (start 128.194 87.046) (end 128.194 76.886) (width 0.5) (layer "B.Cu") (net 45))
 (segment (start 128.194 87.046) (end 133.02 87.046) (width 0.5) (layer "B.Cu") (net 45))
 (segment (start 128.194 76.886) (end 130.734 74.346) (width 0.5) (layer "B.Cu") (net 45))
 (segment (start 122.86 92.38) (end 128.194 87.046) (width 0.5) (layer "B.Cu") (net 45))
 (segment (start 130.734 74.346) (end 133.02 74.346) (width 0.5) (layer "B.Cu") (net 45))
 (segment (start 166.04 74.6) (end 173.66 66.98) (width 0.25) (layer "F.Cu") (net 56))
 (segment (start 141.37 95.068299) (end 161.838299 74.6) (width 0.25) (layer "F.Cu") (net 56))
 (segment (start 173.66 64.44) (end 175.44 62.66) (width 0.25) (layer "F.Cu") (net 56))
 (segment (start 140.005 98.095) (end 141.37 96.73) (width 0.25) (layer "F.Cu") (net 56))
 (segment (start 175.44 62.66) (end 178.74 62.66) (width 0.25) (layer "F.Cu") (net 56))
 (segment (start 141.37 96.73) (end 141.37 95.068299) (width 0.25) (layer "F.Cu") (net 56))
 (segment (start 161.838299 74.6) (end 166.04 74.6) (width 0.25) (layer "F.Cu") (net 56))
 (segment (start 173.66 66.98) (end 173.66 64.44) (width 0.25) (layer "F.Cu") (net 56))
 (segment (start 149.678299 94.38) (end 148.99 95.068299) (width 0.25) (layer "F.Cu") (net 60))
 (segment (start 146.45 96.73) (end 145.085 98.095) (width 0.25) (layer "F.Cu") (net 60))
 (segment (start 181.28 72.62) (end 159.52 94.38) (width 0.25) (layer "F.Cu") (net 60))
 (segment (start 148.99 95.851701) (end 148.111701 96.73) (width 0.25) (layer "F.Cu") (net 60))
 (segment (start 159.52 94.38) (end 149.678299 94.38) (width 0.25) (layer "F.Cu") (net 60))
 (segment (start 148.111701 96.73) (end 146.45 96.73) (width 0.25) (layer "F.Cu") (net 60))
 (segment (start 148.99 95.068299) (end 148.99 95.851701) (width 0.25) (layer "F.Cu") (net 60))
 (segment (start 179.49 64.66) (end 181.28 66.45) (width 0.25) (layer "F.Cu") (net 60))
 (segment (start 181.28 66.45) (end 181.28 72.62) (width 0.25) (layer "F.Cu") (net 60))
 (segment (start 178.74 64.66) (end 179.49 64.66) (width 0.25) (layer "F.Cu") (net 60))
 (segment (start 178.74 66.66) (end 177.99 66.66) (width 0.25) (layer "F.Cu") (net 61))
 (segment (start 152.27 92.38) (end 148.26 92.38) (width 0.25) (layer "F.Cu") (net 61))
 (segment (start 177.99 66.66) (end 152.27 92.38) (width 0.25) (layer "F.Cu") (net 61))
 (segment (start 148.26 92.38) (end 145.085 95.555) (width 0.25) (layer "F.Cu") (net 61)))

